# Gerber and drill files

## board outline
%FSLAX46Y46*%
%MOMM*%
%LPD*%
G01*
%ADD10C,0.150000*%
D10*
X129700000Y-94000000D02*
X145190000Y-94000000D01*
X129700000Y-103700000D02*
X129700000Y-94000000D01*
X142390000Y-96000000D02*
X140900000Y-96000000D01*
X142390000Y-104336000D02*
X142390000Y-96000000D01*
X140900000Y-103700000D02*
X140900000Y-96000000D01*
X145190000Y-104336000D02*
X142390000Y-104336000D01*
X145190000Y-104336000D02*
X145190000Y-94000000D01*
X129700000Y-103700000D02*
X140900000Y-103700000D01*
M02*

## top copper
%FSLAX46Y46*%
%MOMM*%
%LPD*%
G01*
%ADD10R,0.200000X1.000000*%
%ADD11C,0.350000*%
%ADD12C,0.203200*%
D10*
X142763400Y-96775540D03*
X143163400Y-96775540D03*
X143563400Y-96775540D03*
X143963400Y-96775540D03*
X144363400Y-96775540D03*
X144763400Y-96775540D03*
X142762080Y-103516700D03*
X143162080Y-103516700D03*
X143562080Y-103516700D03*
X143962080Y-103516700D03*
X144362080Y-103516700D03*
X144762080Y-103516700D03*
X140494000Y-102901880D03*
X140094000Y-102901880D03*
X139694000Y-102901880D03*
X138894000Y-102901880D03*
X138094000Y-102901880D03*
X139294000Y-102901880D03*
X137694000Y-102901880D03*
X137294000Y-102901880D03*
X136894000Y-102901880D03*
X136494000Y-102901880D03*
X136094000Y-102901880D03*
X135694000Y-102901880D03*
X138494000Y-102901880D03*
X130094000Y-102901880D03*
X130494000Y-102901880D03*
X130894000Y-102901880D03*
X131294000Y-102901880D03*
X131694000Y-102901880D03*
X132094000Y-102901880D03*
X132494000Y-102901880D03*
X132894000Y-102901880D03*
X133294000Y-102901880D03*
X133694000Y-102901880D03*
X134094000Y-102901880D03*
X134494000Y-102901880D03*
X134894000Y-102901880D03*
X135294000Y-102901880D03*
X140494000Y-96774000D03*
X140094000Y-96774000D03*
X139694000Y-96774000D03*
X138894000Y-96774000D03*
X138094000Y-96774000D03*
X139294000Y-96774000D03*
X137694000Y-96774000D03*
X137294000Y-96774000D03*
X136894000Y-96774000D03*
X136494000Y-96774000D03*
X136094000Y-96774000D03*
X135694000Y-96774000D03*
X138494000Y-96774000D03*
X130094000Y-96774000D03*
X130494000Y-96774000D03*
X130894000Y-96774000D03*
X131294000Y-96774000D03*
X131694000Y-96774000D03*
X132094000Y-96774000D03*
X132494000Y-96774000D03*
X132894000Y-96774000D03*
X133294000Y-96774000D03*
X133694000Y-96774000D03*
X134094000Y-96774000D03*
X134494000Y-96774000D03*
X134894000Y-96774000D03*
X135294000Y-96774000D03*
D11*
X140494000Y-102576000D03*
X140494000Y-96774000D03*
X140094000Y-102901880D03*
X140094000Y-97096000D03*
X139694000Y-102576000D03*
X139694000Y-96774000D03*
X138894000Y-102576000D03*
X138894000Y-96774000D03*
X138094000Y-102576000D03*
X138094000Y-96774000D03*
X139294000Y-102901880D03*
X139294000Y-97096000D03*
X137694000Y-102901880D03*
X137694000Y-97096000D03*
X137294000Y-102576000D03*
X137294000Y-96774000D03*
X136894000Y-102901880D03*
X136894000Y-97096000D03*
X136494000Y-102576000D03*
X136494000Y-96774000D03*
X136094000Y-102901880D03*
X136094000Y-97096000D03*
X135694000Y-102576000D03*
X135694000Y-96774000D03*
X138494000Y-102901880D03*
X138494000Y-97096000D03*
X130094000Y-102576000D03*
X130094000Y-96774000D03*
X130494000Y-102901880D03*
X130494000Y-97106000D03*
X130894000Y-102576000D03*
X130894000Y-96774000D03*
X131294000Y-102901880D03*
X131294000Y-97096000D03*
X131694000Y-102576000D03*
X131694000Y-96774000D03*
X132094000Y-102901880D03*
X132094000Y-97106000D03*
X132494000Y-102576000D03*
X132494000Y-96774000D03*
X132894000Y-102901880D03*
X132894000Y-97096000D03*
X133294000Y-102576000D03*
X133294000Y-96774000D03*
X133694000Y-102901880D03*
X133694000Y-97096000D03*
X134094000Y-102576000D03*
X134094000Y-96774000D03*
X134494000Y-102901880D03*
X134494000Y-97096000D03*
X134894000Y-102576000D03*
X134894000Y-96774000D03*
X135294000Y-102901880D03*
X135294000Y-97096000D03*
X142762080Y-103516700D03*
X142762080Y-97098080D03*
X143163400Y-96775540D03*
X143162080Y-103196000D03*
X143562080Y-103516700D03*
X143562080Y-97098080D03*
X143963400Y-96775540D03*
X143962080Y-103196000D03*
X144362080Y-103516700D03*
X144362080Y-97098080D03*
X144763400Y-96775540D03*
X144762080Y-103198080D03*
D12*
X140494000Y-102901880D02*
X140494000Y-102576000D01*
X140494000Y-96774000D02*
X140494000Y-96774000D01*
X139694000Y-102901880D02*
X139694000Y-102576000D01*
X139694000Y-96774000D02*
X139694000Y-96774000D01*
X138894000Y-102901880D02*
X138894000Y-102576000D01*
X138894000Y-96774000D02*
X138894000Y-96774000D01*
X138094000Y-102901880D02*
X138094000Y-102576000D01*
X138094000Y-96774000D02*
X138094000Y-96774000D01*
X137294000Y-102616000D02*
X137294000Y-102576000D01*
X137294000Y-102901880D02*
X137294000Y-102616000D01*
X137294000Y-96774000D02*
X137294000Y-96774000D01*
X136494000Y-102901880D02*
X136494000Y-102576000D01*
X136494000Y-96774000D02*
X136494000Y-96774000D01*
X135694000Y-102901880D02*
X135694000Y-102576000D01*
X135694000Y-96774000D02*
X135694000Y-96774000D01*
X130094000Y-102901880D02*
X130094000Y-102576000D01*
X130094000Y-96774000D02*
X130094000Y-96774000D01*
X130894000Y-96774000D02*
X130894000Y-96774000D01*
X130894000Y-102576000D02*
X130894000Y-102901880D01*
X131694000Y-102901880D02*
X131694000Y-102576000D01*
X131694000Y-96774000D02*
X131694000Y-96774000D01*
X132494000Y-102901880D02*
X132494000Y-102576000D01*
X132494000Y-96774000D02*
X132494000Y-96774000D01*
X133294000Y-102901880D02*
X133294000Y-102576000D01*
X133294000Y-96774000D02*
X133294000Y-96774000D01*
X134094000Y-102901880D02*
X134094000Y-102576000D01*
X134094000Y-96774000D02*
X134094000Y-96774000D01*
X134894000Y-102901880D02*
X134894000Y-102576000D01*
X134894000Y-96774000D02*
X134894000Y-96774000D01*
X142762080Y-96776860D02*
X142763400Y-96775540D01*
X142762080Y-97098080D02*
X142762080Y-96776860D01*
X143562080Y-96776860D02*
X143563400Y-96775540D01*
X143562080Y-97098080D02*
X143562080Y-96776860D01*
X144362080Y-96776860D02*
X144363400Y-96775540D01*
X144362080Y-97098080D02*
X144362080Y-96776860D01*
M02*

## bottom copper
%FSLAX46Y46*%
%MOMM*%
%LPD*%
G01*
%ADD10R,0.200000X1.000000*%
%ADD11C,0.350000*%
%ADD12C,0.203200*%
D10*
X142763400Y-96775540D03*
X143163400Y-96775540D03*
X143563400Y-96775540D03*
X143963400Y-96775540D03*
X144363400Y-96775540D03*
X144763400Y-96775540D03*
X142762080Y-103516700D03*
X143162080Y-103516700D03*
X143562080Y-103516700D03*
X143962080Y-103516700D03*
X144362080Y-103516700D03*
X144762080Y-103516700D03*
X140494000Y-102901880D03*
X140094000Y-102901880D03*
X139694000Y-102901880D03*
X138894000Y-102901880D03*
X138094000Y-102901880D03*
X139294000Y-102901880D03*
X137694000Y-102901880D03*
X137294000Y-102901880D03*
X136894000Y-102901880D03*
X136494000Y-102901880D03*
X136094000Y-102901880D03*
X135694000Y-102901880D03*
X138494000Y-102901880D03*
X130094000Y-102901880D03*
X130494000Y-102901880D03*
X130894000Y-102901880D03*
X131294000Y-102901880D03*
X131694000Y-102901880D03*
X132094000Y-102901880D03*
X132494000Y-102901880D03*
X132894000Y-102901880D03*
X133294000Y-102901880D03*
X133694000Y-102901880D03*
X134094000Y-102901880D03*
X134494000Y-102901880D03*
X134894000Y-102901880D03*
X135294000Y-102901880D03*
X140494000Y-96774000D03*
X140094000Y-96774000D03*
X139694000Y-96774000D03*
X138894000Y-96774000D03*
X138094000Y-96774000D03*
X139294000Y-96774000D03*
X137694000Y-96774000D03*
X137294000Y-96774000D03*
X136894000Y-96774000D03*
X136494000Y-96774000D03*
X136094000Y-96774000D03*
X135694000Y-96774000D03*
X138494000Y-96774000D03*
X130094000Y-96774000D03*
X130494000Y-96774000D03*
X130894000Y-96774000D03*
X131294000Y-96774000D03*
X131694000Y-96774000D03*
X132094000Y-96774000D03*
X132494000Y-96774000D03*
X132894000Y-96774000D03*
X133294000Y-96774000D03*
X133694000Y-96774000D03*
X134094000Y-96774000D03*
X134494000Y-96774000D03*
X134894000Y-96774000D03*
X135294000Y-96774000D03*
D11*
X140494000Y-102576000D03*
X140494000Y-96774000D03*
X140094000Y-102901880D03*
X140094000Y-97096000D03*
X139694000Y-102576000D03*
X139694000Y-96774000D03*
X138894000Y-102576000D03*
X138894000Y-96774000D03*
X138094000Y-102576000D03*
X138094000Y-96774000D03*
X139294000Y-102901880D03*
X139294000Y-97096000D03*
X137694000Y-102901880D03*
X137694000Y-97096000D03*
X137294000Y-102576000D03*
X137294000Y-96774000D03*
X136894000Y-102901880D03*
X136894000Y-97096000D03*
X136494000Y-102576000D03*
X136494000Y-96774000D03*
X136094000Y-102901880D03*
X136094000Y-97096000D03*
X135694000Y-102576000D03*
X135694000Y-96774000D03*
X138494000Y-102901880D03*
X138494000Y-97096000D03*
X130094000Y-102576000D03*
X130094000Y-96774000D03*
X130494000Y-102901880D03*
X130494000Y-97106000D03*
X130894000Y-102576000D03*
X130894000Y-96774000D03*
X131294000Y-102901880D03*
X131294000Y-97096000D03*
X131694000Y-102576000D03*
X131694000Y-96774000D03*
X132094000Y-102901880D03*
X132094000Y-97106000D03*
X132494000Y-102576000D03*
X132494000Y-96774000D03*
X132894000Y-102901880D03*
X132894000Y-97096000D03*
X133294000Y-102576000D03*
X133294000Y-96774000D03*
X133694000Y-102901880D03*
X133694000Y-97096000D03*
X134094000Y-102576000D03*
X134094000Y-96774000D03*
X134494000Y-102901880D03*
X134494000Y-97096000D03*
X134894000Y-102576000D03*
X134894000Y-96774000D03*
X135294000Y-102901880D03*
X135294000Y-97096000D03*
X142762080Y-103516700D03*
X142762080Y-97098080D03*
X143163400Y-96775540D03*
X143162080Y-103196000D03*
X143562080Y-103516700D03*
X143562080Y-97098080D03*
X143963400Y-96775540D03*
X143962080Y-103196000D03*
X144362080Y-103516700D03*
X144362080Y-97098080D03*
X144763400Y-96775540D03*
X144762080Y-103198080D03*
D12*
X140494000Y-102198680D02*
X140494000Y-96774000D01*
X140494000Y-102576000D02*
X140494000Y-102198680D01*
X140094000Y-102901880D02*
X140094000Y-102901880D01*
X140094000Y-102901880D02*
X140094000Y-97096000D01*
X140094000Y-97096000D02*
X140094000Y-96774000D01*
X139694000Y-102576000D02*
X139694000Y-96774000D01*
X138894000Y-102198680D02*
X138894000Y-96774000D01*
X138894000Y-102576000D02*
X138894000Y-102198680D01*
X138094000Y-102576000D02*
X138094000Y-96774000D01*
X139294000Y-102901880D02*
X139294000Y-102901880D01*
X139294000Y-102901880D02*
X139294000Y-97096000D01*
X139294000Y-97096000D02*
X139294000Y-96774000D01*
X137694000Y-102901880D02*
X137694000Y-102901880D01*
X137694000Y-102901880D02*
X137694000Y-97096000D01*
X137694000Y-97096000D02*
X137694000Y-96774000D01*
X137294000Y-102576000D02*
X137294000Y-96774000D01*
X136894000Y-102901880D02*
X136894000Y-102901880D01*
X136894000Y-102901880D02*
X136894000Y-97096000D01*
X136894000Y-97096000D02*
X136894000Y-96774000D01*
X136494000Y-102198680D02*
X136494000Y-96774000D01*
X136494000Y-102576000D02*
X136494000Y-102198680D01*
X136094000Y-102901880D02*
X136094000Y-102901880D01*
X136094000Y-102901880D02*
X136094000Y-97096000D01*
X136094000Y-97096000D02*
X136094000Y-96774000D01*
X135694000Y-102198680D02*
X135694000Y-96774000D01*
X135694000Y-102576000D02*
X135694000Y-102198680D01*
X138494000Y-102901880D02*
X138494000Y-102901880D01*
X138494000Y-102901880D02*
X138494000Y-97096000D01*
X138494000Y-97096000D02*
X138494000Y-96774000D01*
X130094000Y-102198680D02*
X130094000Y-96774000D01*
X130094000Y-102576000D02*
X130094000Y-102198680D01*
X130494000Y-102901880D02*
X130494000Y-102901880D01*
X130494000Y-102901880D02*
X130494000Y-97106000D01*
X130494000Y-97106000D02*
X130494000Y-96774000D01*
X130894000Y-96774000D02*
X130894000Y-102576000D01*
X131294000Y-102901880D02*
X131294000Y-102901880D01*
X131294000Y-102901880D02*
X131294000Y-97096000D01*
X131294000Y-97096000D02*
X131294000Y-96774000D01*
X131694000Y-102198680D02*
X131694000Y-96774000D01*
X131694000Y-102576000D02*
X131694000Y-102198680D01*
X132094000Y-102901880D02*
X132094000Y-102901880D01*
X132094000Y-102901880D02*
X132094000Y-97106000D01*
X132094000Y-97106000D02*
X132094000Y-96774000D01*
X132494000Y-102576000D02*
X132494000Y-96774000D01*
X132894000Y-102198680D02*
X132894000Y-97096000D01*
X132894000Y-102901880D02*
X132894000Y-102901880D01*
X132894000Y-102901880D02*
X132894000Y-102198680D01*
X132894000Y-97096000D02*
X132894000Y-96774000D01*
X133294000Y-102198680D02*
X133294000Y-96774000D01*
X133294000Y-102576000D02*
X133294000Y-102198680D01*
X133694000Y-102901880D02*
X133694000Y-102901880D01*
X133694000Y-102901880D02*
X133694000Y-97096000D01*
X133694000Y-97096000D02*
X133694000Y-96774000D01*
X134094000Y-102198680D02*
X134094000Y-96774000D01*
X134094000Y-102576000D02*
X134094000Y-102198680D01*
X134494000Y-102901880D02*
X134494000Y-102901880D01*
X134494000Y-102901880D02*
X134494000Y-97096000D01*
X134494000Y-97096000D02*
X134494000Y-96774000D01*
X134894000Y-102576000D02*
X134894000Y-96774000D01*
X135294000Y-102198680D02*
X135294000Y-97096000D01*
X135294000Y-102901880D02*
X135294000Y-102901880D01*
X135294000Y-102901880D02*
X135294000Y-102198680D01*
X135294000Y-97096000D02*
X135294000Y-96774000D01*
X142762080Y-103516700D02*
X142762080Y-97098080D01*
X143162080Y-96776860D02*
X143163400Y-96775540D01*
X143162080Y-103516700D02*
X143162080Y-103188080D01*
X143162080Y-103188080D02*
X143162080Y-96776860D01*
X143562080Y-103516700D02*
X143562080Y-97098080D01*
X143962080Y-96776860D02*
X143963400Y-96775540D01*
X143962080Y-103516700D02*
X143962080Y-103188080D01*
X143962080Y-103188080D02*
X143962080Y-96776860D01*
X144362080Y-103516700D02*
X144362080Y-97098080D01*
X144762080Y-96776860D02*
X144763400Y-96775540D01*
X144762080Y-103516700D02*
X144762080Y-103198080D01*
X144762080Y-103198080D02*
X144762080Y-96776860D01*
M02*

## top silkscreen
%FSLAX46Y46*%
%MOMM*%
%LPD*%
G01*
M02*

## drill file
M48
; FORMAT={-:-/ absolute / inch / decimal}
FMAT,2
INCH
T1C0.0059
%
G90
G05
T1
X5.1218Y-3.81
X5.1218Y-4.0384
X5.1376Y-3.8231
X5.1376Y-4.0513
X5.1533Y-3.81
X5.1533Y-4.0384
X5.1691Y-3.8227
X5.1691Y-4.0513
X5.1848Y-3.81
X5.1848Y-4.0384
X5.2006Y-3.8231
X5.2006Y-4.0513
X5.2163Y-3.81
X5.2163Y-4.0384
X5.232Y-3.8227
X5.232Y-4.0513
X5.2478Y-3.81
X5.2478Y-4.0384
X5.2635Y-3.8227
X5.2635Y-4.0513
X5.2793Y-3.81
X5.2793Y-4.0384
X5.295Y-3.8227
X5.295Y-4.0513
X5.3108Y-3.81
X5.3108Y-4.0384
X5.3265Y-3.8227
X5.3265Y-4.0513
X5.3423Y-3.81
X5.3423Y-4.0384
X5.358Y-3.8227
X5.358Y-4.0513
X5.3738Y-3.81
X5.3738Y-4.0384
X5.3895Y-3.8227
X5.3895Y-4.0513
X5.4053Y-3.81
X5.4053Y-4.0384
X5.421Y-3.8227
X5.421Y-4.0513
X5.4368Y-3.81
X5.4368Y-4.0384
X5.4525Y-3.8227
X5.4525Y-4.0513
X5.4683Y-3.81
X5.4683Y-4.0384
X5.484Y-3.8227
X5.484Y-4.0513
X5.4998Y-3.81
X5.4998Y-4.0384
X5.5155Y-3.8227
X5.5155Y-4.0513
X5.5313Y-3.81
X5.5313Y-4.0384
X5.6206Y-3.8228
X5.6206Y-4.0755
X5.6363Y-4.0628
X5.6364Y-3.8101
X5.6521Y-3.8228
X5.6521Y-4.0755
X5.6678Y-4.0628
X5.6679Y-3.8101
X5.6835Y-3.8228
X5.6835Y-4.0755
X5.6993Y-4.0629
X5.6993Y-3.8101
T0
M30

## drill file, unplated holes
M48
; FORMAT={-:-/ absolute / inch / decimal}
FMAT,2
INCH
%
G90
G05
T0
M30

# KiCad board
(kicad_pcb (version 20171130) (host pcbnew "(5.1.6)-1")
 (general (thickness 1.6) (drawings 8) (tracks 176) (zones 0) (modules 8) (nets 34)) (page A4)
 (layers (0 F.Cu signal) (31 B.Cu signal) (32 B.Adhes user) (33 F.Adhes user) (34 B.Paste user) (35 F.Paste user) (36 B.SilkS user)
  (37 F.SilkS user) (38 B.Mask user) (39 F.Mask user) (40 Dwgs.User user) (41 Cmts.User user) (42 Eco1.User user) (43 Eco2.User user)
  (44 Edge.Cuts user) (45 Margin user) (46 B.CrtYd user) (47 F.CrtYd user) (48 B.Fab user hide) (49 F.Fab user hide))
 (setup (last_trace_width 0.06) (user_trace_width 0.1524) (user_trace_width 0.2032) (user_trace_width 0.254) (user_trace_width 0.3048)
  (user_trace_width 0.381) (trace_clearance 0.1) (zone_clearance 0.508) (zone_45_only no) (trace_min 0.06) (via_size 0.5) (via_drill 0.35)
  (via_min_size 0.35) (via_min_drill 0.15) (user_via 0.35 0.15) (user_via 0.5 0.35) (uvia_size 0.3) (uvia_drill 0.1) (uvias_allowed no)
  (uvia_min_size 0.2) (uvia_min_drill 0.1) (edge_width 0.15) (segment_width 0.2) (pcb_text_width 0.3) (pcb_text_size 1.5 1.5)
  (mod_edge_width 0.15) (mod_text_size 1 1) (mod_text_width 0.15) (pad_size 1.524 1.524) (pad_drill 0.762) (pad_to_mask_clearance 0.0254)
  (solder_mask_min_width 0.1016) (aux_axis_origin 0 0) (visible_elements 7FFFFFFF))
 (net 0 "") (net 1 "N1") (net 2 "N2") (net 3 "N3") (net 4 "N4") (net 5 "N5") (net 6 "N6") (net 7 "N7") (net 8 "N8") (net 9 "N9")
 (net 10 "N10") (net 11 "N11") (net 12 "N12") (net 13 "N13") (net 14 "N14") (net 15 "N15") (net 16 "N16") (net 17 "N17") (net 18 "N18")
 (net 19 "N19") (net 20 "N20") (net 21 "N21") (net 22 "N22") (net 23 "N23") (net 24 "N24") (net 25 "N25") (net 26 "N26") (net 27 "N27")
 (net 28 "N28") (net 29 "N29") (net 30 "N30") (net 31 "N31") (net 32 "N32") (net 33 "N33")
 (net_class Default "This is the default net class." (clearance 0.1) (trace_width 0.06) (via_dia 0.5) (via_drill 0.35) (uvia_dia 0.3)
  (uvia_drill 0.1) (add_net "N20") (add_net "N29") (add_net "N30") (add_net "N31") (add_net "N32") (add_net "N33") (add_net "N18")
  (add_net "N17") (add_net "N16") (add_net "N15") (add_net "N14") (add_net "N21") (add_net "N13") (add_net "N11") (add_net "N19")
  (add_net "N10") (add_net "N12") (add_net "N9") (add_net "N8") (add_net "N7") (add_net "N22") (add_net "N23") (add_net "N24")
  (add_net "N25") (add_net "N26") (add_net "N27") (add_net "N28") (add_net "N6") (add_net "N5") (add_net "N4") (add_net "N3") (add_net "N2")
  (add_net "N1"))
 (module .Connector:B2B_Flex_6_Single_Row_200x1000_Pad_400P (layer F.Cu) (at 144.7634 96.77554 180)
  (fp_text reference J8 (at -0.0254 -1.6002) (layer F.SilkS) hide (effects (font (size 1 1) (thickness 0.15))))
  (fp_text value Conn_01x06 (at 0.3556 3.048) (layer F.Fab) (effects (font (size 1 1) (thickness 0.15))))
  (pad 6 smd rect (at 2 0 180) (size 0.2 1) (layers F.Cu F.Paste F.Mask) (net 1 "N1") (zone_connect 0))
  (pad 5 smd rect (at 1.6 0 180) (size 0.2 1) (layers F.Cu F.Paste F.Mask) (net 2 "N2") (zone_connect 0))
  (pad 4 smd rect (at 1.2 0 180) (size 0.2 1) (layers F.Cu F.Paste F.Mask) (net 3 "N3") (zone_connect 0))
  (pad 3 smd rect (at 0.8 0 180) (size 0.2 1) (layers F.Cu F.Paste F.Mask) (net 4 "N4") (zone_connect 0))
  (pad 2 smd rect (at 0.4 0 180) (size 0.2 1) (layers F.Cu F.Paste F.Mask) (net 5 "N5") (zone_connect 0))
  (pad 1 smd rect (at 0 0 180) (size 0.2 1) (layers F.Cu F.Paste F.Mask) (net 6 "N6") (zone_connect 0)))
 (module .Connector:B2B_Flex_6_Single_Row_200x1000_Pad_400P (layer F.Cu) (at 144.76208 103.5167 180)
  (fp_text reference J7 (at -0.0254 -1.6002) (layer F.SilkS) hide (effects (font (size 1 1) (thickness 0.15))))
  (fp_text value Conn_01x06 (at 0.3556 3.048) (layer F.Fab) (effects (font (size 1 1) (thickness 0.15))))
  (pad 6 smd rect (at 2 0 180) (size 0.2 1) (layers F.Cu F.Paste F.Mask) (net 1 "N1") (zone_connect 0))
  (pad 5 smd rect (at 1.6 0 180) (size 0.2 1) (layers F.Cu F.Paste F.Mask) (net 2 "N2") (zone_connect 0))
  (pad 4 smd rect (at 1.2 0 180) (size 0.2 1) (layers F.Cu F.Paste F.Mask) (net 3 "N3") (zone_connect 0))
  (pad 3 smd rect (at 0.8 0 180) (size 0.2 1) (layers F.Cu F.Paste F.Mask) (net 4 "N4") (zone_connect 0))
  (pad 2 smd rect (at 0.4 0 180) (size 0.2 1) (layers F.Cu F.Paste F.Mask) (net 5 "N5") (zone_connect 0))
  (pad 1 smd rect (at 0 0 180) (size 0.2 1) (layers F.Cu F.Paste F.Mask) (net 6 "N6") (zone_connect 0)))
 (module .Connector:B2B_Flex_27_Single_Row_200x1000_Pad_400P (layer F.Cu) (at 130.094 102.90188)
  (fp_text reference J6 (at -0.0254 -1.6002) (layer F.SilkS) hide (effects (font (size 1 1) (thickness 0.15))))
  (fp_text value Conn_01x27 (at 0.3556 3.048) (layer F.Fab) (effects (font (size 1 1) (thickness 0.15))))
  (pad 27 smd rect (at 10.4 0) (size 0.2 1) (layers F.Cu F.Paste F.Mask) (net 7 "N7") (zone_connect 0))
  (pad 26 smd rect (at 10 0) (size 0.2 1) (layers F.Cu F.Paste F.Mask) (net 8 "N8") (zone_connect 0))
  (pad 25 smd rect (at 9.6 0) (size 0.2 1) (layers F.Cu F.Paste F.Mask) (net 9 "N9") (zone_connect 0))
  (pad 23 smd rect (at 8.8 0) (size 0.2 1) (layers F.Cu F.Paste F.Mask) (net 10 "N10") (zone_connect 0))
  (pad 21 smd rect (at 8 0) (size 0.2 1) (layers F.Cu F.Paste F.Mask) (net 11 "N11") (zone_connect 0))
  (pad 24 smd rect (at 9.2 0) (size 0.2 1) (layers F.Cu F.Paste F.Mask) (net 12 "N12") (zone_connect 0))
  (pad 20 smd rect (at 7.6 0) (size 0.2 1) (layers F.Cu F.Paste F.Mask) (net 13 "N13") (zone_connect 0))
  (pad 19 smd rect (at 7.2 0) (size 0.2 1) (layers F.Cu F.Paste F.Mask) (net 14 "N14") (zone_connect 0))
  (pad 18 smd rect (at 6.8 0) (size 0.2 1) (layers F.Cu F.Paste F.Mask) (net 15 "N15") (zone_connect 0))
  (pad 17 smd rect (at 6.4 0) (size 0.2 1) (layers F.Cu F.Paste F.Mask) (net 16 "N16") (zone_connect 0))
  (pad 16 smd rect (at 6 0) (size 0.2 1) (layers F.Cu F.Paste F.Mask) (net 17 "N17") (zone_connect 0))
  (pad 15 smd rect (at 5.6 0) (size 0.2 1) (layers F.Cu F.Paste F.Mask) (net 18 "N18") (zone_connect 0))
  (pad 22 smd rect (at 8.4 0) (size 0.2 1) (layers F.Cu F.Paste F.Mask) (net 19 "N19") (zone_connect 0))
  (pad 1 smd rect (at 0 0) (size 0.2 1) (layers F.Cu F.Paste F.Mask) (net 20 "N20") (zone_connect 0))
  (pad 2 smd rect (at 0.4 0) (size 0.2 1) (layers F.Cu F.Paste F.Mask) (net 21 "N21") (zone_connect 0))
  (pad 3 smd rect (at 0.8 0) (size 0.2 1) (layers F.Cu F.Paste F.Mask) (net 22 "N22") (zone_connect 0))
  (pad 4 smd rect (at 1.2 0) (size 0.2 1) (layers F.Cu F.Paste F.Mask) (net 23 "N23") (zone_connect 0))
  (pad 5 smd rect (at 1.6 0) (size 0.2 1) (layers F.Cu F.Paste F.Mask) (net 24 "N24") (zone_connect 0))
  (pad 6 smd rect (at 2 0) (size 0.2 1) (layers F.Cu F.Paste F.Mask) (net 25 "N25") (zone_connect 0))
  (pad 7 smd rect (at 2.4 0) (size 0.2 1) (layers F.Cu F.Paste F.Mask) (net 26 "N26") (zone_connect 0))
  (pad 8 smd rect (at 2.8 0) (size 0.2 1) (layers F.Cu F.Paste F.Mask) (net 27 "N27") (zone_connect 0))
  (pad 9 smd rect (at 3.2 0) (size 0.2 1) (layers F.Cu F.Paste F.Mask) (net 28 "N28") (zone_connect 0))
  (pad 10 smd rect (at 3.6 0) (size 0.2 1) (layers F.Cu F.Paste F.Mask) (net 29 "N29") (zone_connect 0))
  (pad 11 smd rect (at 4 0) (size 0.2 1) (layers F.Cu F.Paste F.Mask) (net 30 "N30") (zone_connect 0))
  (pad 12 smd rect (at 4.4 0) (size 0.2 1) (layers F.Cu F.Paste F.Mask) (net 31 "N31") (zone_connect 0))
  (pad 13 smd rect (at 4.8 0) (size 0.2 1) (layers F.Cu F.Paste F.Mask) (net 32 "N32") (zone_connect 0))
  (pad 14 smd rect (at 5.2 0) (size 0.2 1) (layers F.Cu F.Paste F.Mask) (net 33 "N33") (zone_connect 0)))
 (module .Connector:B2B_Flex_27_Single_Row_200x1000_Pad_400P (layer F.Cu) (at 130.094 96.774)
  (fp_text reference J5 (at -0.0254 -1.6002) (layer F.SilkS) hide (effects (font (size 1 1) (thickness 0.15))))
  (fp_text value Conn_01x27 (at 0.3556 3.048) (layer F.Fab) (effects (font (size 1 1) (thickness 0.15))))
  (pad 27 smd rect (at 10.4 0) (size 0.2 1) (layers F.Cu F.Paste F.Mask) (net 7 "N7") (zone_connect 0))
  (pad 26 smd rect (at 10 0) (size 0.2 1) (layers F.Cu F.Paste F.Mask) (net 8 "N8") (zone_connect 0))
  (pad 25 smd rect (at 9.6 0) (size 0.2 1) (layers F.Cu F.Paste F.Mask) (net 9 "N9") (zone_connect 0))
  (pad 23 smd rect (at 8.8 0) (size 0.2 1) (layers F.Cu F.Paste F.Mask) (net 10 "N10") (zone_connect 0))
  (pad 21 smd rect (at 8 0) (size 0.2 1) (layers F.Cu F.Paste F.Mask) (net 11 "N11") (zone_connect 0))
  (pad 24 smd rect (at 9.2 0) (size 0.2 1) (layers F.Cu F.Paste F.Mask) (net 12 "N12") (zone_connect 0))
  (pad 20 smd rect (at 7.6 0) (size 0.2 1) (layers F.Cu F.Paste F.Mask) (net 13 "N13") (zone_connect 0))
  (pad 19 smd rect (at 7.2 0) (size 0.2 1) (layers F.Cu F.Paste F.Mask) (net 14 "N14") (zone_connect 0))
  (pad 18 smd rect (at 6.8 0) (size 0.2 1) (layers F.Cu F.Paste F.Mask) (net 15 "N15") (zone_connect 0))
  (pad 17 smd rect (at 6.4 0) (size 0.2 1) (layers F.Cu F.Paste F.Mask) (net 16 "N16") (zone_connect 0))
  (pad 16 smd rect (at 6 0) (size 0.2 1) (layers F.Cu F.Paste F.Mask) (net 17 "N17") (zone_connect 0))
  (pad 15 smd rect (at 5.6 0) (size 0.2 1) (layers F.Cu F.Paste F.Mask) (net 18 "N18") (zone_connect 0))
  (pad 22 smd rect (at 8.4 0) (size 0.2 1) (layers F.Cu F.Paste F.Mask) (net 19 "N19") (zone_connect 0))
  (pad 1 smd rect (at 0 0) (size 0.2 1) (layers F.Cu F.Paste F.Mask) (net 20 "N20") (zone_connect 0))
  (pad 2 smd rect (at 0.4 0) (size 0.2 1) (layers F.Cu F.Paste F.Mask) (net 21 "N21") (zone_connect 0))
  (pad 3 smd rect (at 0.8 0) (size 0.2 1) (layers F.Cu F.Paste F.Mask) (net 22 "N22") (zone_connect 0))
  (pad 4 smd rect (at 1.2 0) (size 0.2 1) (layers F.Cu F.Paste F.Mask) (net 23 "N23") (zone_connect 0))
  (pad 5 smd rect (at 1.6 0) (size 0.2 1) (layers F.Cu F.Paste F.Mask) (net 24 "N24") (zone_connect 0))
  (pad 6 smd rect (at 2 0) (size 0.2 1) (layers F.Cu F.Paste F.Mask) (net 25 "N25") (zone_connect 0))
  (pad 7 smd rect (at 2.4 0) (size 0.2 1) (layers F.Cu F.Paste F.Mask) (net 26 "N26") (zone_connect 0))
  (pad 8 smd rect (at 2.8 0) (size 0.2 1) (layers F.Cu F.Paste F.Mask) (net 27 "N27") (zone_connect 0))
  (pad 9 smd rect (at 3.2 0) (size 0.2 1) (layers F.Cu F.Paste F.Mask) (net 28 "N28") (zone_connect 0))
  (pad 10 smd rect (at 3.6 0) (size 0.2 1) (layers F.Cu F.Paste F.Mask) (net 29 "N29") (zone_connect 0))
  (pad 11 smd rect (at 4 0) (size 0.2 1) (layers F.Cu F.Paste F.Mask) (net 30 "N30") (zone_connect 0))
  (pad 12 smd rect (at 4.4 0) (size 0.2 1) (layers F.Cu F.Paste F.Mask) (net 31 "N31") (zone_connect 0))
  (pad 13 smd rect (at 4.8 0) (size 0.2 1) (layers F.Cu F.Paste F.Mask) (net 32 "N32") (zone_connect 0))
  (pad 14 smd rect (at 5.2 0) (size 0.2 1) (layers F.Cu F.Paste F.Mask) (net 33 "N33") (zone_connect 0)))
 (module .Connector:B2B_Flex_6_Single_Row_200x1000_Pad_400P (layer B.Cu) (at 144.7634 96.77554 180)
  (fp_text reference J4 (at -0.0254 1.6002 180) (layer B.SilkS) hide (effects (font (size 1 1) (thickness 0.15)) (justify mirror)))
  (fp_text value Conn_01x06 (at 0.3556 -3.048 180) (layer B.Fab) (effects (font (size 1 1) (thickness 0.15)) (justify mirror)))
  (pad 6 smd rect (at 2 0 180) (size 0.2 1) (layers B.Cu B.Paste B.Mask) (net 1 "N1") (zone_connect 0))
  (pad 5 smd rect (at 1.6 0 180) (size 0.2 1) (layers B.Cu B.Paste B.Mask) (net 2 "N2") (zone_connect 0))
  (pad 4 smd rect (at 1.2 0 180) (size 0.2 1) (layers B.Cu B.Paste B.Mask) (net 3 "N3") (zone_connect 0))
  (pad 3 smd rect (at 0.8 0 180) (size 0.2 1) (layers B.Cu B.Paste B.Mask) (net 4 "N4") (zone_connect 0))
  (pad 2 smd rect (at 0.4 0 180) (size 0.2 1) (layers B.Cu B.Paste B.Mask) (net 5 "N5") (zone_connect 0))
  (pad 1 smd rect (at 0 0 180) (size 0.2 1) (layers B.Cu B.Paste B.Mask) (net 6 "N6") (zone_connect 0)))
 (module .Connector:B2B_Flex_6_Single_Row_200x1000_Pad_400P (layer B.Cu) (at 144.76208 103.5167 180)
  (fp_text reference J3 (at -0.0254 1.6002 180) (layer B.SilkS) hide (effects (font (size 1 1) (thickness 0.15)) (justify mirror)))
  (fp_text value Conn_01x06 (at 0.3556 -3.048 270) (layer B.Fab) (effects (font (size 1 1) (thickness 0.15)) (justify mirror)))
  (pad 6 smd rect (at 2 0 180) (size 0.2 1) (layers B.Cu B.Paste B.Mask) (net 1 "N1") (zone_connect 0))
  (pad 5 smd rect (at 1.6 0 180) (size 0.2 1) (layers B.Cu B.Paste B.Mask) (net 2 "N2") (zone_connect 0))
  (pad 4 smd rect (at 1.2 0 180) (size 0.2 1) (layers B.Cu B.Paste B.Mask) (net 3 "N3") (zone_connect 0))
  (pad 3 smd rect (at 0.8 0 180) (size 0.2 1) (layers B.Cu B.Paste B.Mask) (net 4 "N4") (zone_connect 0))
  (pad 2 smd rect (at 0.4 0 180) (size 0.2 1) (layers B.Cu B.Paste B.Mask) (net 5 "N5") (zone_connect 0))
  (pad 1 smd rect (at 0 0 180) (size 0.2 1) (layers B.Cu B.Paste B.Mask) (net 6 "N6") (zone_connect 0)))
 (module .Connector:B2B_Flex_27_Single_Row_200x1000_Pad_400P (layer B.Cu) (at 130.094 102.90188)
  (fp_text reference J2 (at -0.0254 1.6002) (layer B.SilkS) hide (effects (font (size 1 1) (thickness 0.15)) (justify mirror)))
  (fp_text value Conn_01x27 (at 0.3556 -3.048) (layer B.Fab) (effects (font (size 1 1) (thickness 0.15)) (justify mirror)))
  (pad 27 smd rect (at 10.4 0) (size 0.2 1) (layers B.Cu B.Paste B.Mask) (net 7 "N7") (zone_connect 0))
  (pad 26 smd rect (at 10 0) (size 0.2 1) (layers B.Cu B.Paste B.Mask) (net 8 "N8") (zone_connect 0))
  (pad 25 smd rect (at 9.6 0) (size 0.2 1) (layers B.Cu B.Paste B.Mask) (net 9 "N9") (zone_connect 0))
  (pad 23 smd rect (at 8.8 0) (size 0.2 1) (layers B.Cu B.Paste B.Mask) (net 10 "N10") (zone_connect 0))
  (pad 21 smd rect (at 8 0) (size 0.2 1) (layers B.Cu B.Paste B.Mask) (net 11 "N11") (zone_connect 0))
  (pad 24 smd rect (at 9.2 0) (size 0.2 1) (layers B.Cu B.Paste B.Mask) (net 12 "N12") (zone_connect 0))
  (pad 20 smd rect (at 7.6 0) (size 0.2 1) (layers B.Cu B.Paste B.Mask) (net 13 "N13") (zone_connect 0))
  (pad 19 smd rect (at 7.2 0) (size 0.2 1) (layers B.Cu B.Paste B.Mask) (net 14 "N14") (zone_connect 0))
  (pad 18 smd rect (at 6.8 0) (size 0.2 1) (layers B.Cu B.Paste B.Mask) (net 15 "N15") (zone_connect 0))
  (pad 17 smd rect (at 6.4 0) (size 0.2 1) (layers B.Cu B.Paste B.Mask) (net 16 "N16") (zone_connect 0))
  (pad 16 smd rect (at 6 0) (size 0.2 1) (layers B.Cu B.Paste B.Mask) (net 17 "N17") (zone_connect 0))
  (pad 15 smd rect (at 5.6 0) (size 0.2 1) (layers B.Cu B.Paste B.Mask) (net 18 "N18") (zone_connect 0))
  (pad 22 smd rect (at 8.4 0) (size 0.2 1) (layers B.Cu B.Paste B.Mask) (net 19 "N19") (zone_connect 0))
  (pad 1 smd rect (at 0 0) (size 0.2 1) (layers B.Cu B.Paste B.Mask) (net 20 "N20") (zone_connect 0))
  (pad 2 smd rect (at 0.4 0) (size 0.2 1) (layers B.Cu B.Paste B.Mask) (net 21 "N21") (zone_connect 0))
  (pad 3 smd rect (at 0.8 0) (size 0.2 1) (layers B.Cu B.Paste B.Mask) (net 22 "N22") (zone_connect 0))
  (pad 4 smd rect (at 1.2 0) (size 0.2 1) (layers B.Cu B.Paste B.Mask) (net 23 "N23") (zone_connect 0))
  (pad 5 smd rect (at 1.6 0) (size 0.2 1) (layers B.Cu B.Paste B.Mask) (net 24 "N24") (zone_connect 0))
  (pad 6 smd rect (at 2 0) (size 0.2 1) (layers B.Cu B.Paste B.Mask) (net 25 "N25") (zone_connect 0))
  (pad 7 smd rect (at 2.4 0) (size 0.2 1) (layers B.Cu B.Paste B.Mask) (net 26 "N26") (zone_connect 0))
  (pad 8 smd rect (at 2.8 0) (size 0.2 1) (layers B.Cu B.Paste B.Mask) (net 27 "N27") (zone_connect 0))
  (pad 9 smd rect (at 3.2 0) (size 0.2 1) (layers B.Cu B.Paste B.Mask) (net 28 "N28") (zone_connect 0))
  (pad 10 smd rect (at 3.6 0) (size 0.2 1) (layers B.Cu B.Paste B.Mask) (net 29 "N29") (zone_connect 0))
  (pad 11 smd rect (at 4 0) (size 0.2 1) (layers B.Cu B.Paste B.Mask) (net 30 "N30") (zone_connect 0))
  (pad 12 smd rect (at 4.4 0) (size 0.2 1) (layers B.Cu B.Paste B.Mask) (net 31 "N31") (zone_connect 0))
  (pad 13 smd rect (at 4.8 0) (size 0.2 1) (layers B.Cu B.Paste B.Mask) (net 32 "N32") (zone_connect 0))
  (pad 14 smd rect (at 5.2 0) (size 0.2 1) (layers B.Cu B.Paste B.Mask) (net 33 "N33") (zone_connect 0)))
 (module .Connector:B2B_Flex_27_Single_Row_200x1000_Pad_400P (layer B.Cu) (at 130.094 96.774)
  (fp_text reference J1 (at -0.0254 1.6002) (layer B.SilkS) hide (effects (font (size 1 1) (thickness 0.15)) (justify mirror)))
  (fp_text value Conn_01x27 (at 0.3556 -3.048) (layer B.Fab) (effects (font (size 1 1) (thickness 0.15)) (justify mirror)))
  (pad 27 smd rect (at 10.4 0) (size 0.2 1) (layers B.Cu B.Paste B.Mask) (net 7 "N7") (zone_connect 0))
  (pad 26 smd rect (at 10 0) (size 0.2 1) (layers B.Cu B.Paste B.Mask) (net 8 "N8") (zone_connect 0))
  (pad 25 smd rect (at 9.6 0) (size 0.2 1) (layers B.Cu B.Paste B.Mask) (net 9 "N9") (zone_connect 0))
  (pad 23 smd rect (at 8.8 0) (size 0.2 1) (layers B.Cu B.Paste B.Mask) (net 10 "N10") (zone_connect 0))
  (pad 21 smd rect (at 8 0) (size 0.2 1) (layers B.Cu B.Paste B.Mask) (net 11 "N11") (zone_connect 0))
  (pad 24 smd rect (at 9.2 0) (size 0.2 1) (layers B.Cu B.Paste B.Mask) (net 12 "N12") (zone_connect 0))
  (pad 20 smd rect (at 7.6 0) (size 0.2 1) (layers B.Cu B.Paste B.Mask) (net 13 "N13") (zone_connect 0))
  (pad 19 smd rect (at 7.2 0) (size 0.2 1) (layers B.Cu B.Paste B.Mask) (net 14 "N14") (zone_connect 0))
  (pad 18 smd rect (at 6.8 0) (size 0.2 1) (layers B.Cu B.Paste B.Mask) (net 15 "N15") (zone_connect 0))
  (pad 17 smd rect (at 6.4 0) (size 0.2 1) (layers B.Cu B.Paste B.Mask) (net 16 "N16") (zone_connect 0))
  (pad 16 smd rect (at 6 0) (size 0.2 1) (layers B.Cu B.Paste B.Mask) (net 17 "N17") (zone_connect 0))
  (pad 15 smd rect (at 5.6 0) (size 0.2 1) (layers B.Cu B.Paste B.Mask) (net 18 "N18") (zone_connect 0))
  (pad 22 smd rect (at 8.4 0) (size 0.2 1) (layers B.Cu B.Paste B.Mask) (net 19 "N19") (zone_connect 0))
  (pad 1 smd rect (at 0 0) (size 0.2 1) (layers B.Cu B.Paste B.Mask) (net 20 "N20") (zone_connect 0))
  (pad 2 smd rect (at 0.4 0) (size 0.2 1) (layers B.Cu B.Paste B.Mask) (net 21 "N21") (zone_connect 0))
  (pad 3 smd rect (at 0.8 0) (size 0.2 1) (layers B.Cu B.Paste B.Mask) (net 22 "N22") (zone_connect 0))
  (pad 4 smd rect (at 1.2 0) (size 0.2 1) (layers B.Cu B.Paste B.Mask) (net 23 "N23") (zone_connect 0))
  (pad 5 smd rect (at 1.6 0) (size 0.2 1) (layers B.Cu B.Paste B.Mask) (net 24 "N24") (zone_connect 0))
  (pad 6 smd rect (at 2 0) (size 0.2 1) (layers B.Cu B.Paste B.Mask) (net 25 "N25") (zone_connect 0))
  (pad 7 smd rect (at 2.4 0) (size 0.2 1) (layers B.Cu B.Paste B.Mask) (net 26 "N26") (zone_connect 0))
  (pad 8 smd rect (at 2.8 0) (size 0.2 1) (layers B.Cu B.Paste B.Mask) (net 27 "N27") (zone_connect 0))
  (pad 9 smd rect (at 3.2 0) (size 0.2 1) (layers B.Cu B.Paste B.Mask) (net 28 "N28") (zone_connect 0))
  (pad 10 smd rect (at 3.6 0) (size 0.2 1) (layers B.Cu B.Paste B.Mask) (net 29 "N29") (zone_connect 0))
  (pad 11 smd rect (at 4 0) (size 0.2 1) (layers B.Cu B.Paste B.Mask) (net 30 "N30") (zone_connect 0))
  (pad 12 smd rect (at 4.4 0) (size 0.2 1) (layers B.Cu B.Paste B.Mask) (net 31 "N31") (zone_connect 0))
  (pad 13 smd rect (at 4.8 0) (size 0.2 1) (layers B.Cu B.Paste B.Mask) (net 32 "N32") (zone_connect 0))
  (pad 14 smd rect (at 5.2 0) (size 0.2 1) (layers B.Cu B.Paste B.Mask) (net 33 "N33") (zone_connect 0)))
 (gr_line (start 129.7 94) (end 145.19 94) (layer Edge.Cuts) (width 0.15))
 (gr_line (start 129.7 103.7) (end 129.7 94) (layer Edge.Cuts) (width 0.15))
 (gr_line (start 142.39 96) (end 140.9 96) (layer Edge.Cuts) (width 0.15))
 (gr_line (start 142.39 104.336) (end 142.39 96) (layer Edge.Cuts) (width 0.15))
 (gr_line (start 140.9 103.7) (end 140.9 96) (layer Edge.Cuts) (width 0.15))
 (gr_line (start 145.19 104.336) (end 142.39 104.336) (layer Edge.Cuts) (width 0.15))
 (gr_line (start 145.19 104.336) (end 145.19 94) (layer Edge.Cuts) (width 0.15))
 (gr_line (start 129.7 103.7) (end 140.9 103.7) (layer Edge.Cuts) (width 0.15))
 (segment (start 140.494 102.19868) (end 140.494 96.774) (width 0.2032) (layer B.Cu) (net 7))
 (segment (start 140.494 102.90188) (end 140.494 102.576) (width 0.2032) (layer F.Cu) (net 7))
 (segment (start 140.494 102.576) (end 140.494 102.19868) (width 0.2032) (layer B.Cu) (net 7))
 (via (at 140.494 102.576) (size 0.35) (drill 0.15) (layers F.Cu B.Cu) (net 7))
 (segment (start 140.494 96.774) (end 140.494 96.774) (width 0.2032) (layer F.Cu) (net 7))
 (via (at 140.494 96.774) (size 0.35) (drill 0.15) (layers F.Cu B.Cu) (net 7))
 (segment (start 140.094 102.90188) (end 140.094 102.90188) (width 0.2032) (layer B.Cu) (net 8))
 (segment (start 140.094 102.90188) (end 140.094 97.096) (width 0.2032) (layer B.Cu) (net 8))
 (via (at 140.094 102.90188) (size 0.35) (drill 0.15) (layers F.Cu B.Cu) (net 8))
 (segment (start 140.094 97.096) (end 140.094 96.774) (width 0.2032) (layer B.Cu) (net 8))
 (via (at 140.094 97.096) (size 0.35) (drill 0.15) (layers F.Cu B.Cu) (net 8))
 (segment (start 139.694 102.90188) (end 139.694 102.576) (width 0.2032) (layer F.Cu) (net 9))
 (segment (start 139.694 102.576) (end 139.694 96.774) (width 0.2032) (layer B.Cu) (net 9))
 (via (at 139.694 102.576) (size 0.35) (drill 0.15) (layers F.Cu B.Cu) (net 9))
 (segment (start 139.694 96.774) (end 139.694 96.774) (width 0.2032) (layer F.Cu) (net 9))
 (via (at 139.694 96.774) (size 0.35) (drill 0.15) (layers F.Cu B.Cu) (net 9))
 (segment (start 138.894 102.19868) (end 138.894 96.774) (width 0.2032) (layer B.Cu) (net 10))
 (segment (start 138.894 102.90188) (end 138.894 102.576) (width 0.2032) (layer F.Cu) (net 10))
 (segment (start 138.894 102.576) (end 138.894 102.19868) (width 0.2032) (layer B.Cu) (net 10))
 (via (at 138.894 102.576) (size 0.35) (drill 0.15) (layers F.Cu B.Cu) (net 10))
 (segment (start 138.894 96.774) (end 138.894 96.774) (width 0.2032) (layer F.Cu) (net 10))
 (via (at 138.894 96.774) (size 0.35) (drill 0.15) (layers F.Cu B.Cu) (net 10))
 (segment (start 138.094 102.90188) (end 138.094 102.576) (width 0.2032) (layer F.Cu) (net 11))
 (segment (start 138.094 102.576) (end 138.094 96.774) (width 0.2032) (layer B.Cu) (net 11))
 (via (at 138.094 102.576) (size 0.35) (drill 0.15) (layers F.Cu B.Cu) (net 11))
 (segment (start 138.094 96.774) (end 138.094 96.774) (width 0.2032) (layer F.Cu) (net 11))
 (via (at 138.094 96.774) (size 0.35) (drill 0.15) (layers F.Cu B.Cu) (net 11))
 (segment (start 139.294 102.90188) (end 139.294 102.90188) (width 0.2032) (layer B.Cu) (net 12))
 (segment (start 139.294 102.90188) (end 139.294 97.096) (width 0.2032) (layer B.Cu) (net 12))
 (via (at 139.294 102.90188) (size 0.35) (drill 0.15) (layers F.Cu B.Cu) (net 12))
 (segment (start 139.294 97.096) (end 139.294 96.774) (width 0.2032) (layer B.Cu) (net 12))
 (via (at 139.294 97.096) (size 0.35) (drill 0.15) (layers F.Cu B.Cu) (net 12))
 (segment (start 137.694 102.90188) (end 137.694 102.90188) (width 0.2032) (layer B.Cu) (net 13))
 (segment (start 137.694 102.90188) (end 137.694 97.096) (width 0.2032) (layer B.Cu) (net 13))
 (via (at 137.694 102.90188) (size 0.35) (drill 0.15) (layers F.Cu B.Cu) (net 13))
 (segment (start 137.694 97.096) (end 137.694 96.774) (width 0.2032) (layer B.Cu) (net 13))
 (via (at 137.694 97.096) (size 0.35) (drill 0.15) (layers F.Cu B.Cu) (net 13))
 (segment (start 137.294 102.616) (end 137.294 102.576) (width 0.2032) (layer F.Cu) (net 14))
 (segment (start 137.294 102.90188) (end 137.294 102.616) (width 0.2032) (layer F.Cu) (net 14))
 (segment (start 137.294 102.576) (end 137.294 96.774) (width 0.2032) (layer B.Cu) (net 14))
 (via (at 137.294 102.576) (size 0.35) (drill 0.15) (layers F.Cu B.Cu) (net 14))
 (segment (start 137.294 96.774) (end 137.294 96.774) (width 0.2032) (layer F.Cu) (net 14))
 (via (at 137.294 96.774) (size 0.35) (drill 0.15) (layers F.Cu B.Cu) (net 14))
 (segment (start 136.894 102.90188) (end 136.894 102.90188) (width 0.2032) (layer B.Cu) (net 15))
 (segment (start 136.894 102.90188) (end 136.894 97.096) (width 0.2032) (layer B.Cu) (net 15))
 (via (at 136.894 102.90188) (size 0.35) (drill 0.15) (layers F.Cu B.Cu) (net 15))
 (segment (start 136.894 97.096) (end 136.894 96.774) (width 0.2032) (layer B.Cu) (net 15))
 (via (at 136.894 97.096) (size 0.35) (drill 0.15) (layers F.Cu B.Cu) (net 15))
 (segment (start 136.494 102.19868) (end 136.494 96.774) (width 0.2032) (layer B.Cu) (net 16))
 (segment (start 136.494 102.90188) (end 136.494 102.576) (width 0.2032) (layer F.Cu) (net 16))
 (segment (start 136.494 102.576) (end 136.494 102.19868) (width 0.2032) (layer B.Cu) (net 16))
 (via (at 136.494 102.576) (size 0.35) (drill 0.15) (layers F.Cu B.Cu) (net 16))
 (segment (start 136.494 96.774) (end 136.494 96.774) (width 0.2032) (layer F.Cu) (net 16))
 (via (at 136.494 96.774) (size 0.35) (drill 0.15) (layers F.Cu B.Cu) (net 16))
 (segment (start 136.094 102.90188) (end 136.094 102.90188) (width 0.2032) (layer B.Cu) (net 17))
 (segment (start 136.094 102.90188) (end 136.094 97.096) (width 0.2032) (layer B.Cu) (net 17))
 (via (at 136.094 102.90188) (size 0.35) (drill 0.15) (layers F.Cu B.Cu) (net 17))
 (segment (start 136.094 97.096) (end 136.094 96.774) (width 0.2032) (layer B.Cu) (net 17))
 (via (at 136.094 97.096) (size 0.35) (drill 0.15) (layers F.Cu B.Cu) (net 17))
 (segment (start 135.694 102.19868) (end 135.694 96.774) (width 0.2032) (layer B.Cu) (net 18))
 (segment (start 135.694 102.90188) (end 135.694 102.576) (width 0.2032) (layer F.Cu) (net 18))
 (segment (start 135.694 102.576) (end 135.694 102.19868) (width 0.2032) (layer B.Cu) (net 18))
 (via (at 135.694 102.576) (size 0.35) (drill 0.15) (layers F.Cu B.Cu) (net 18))
 (segment (start 135.694 96.774) (end 135.694 96.774) (width 0.2032) (layer F.Cu) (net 18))
 (via (at 135.694 96.774) (size 0.35) (drill 0.15) (layers F.Cu B.Cu) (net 18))
 (segment (start 138.494 102.90188) (end 138.494 102.90188) (width 0.2032) (layer B.Cu) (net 19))
 (segment (start 138.494 102.90188) (end 138.494 97.096) (width 0.2032) (layer B.Cu) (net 19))
 (via (at 138.494 102.90188) (size 0.35) (drill 0.15) (layers F.Cu B.Cu) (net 19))
 (segment (start 138.494 97.096) (end 138.494 96.774) (width 0.2032) (layer B.Cu) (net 19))
 (via (at 138.494 97.096) (size 0.35) (drill 0.15) (layers F.Cu B.Cu) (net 19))
 (segment (start 130.094 102.19868) (end 130.094 96.774) (width 0.2032) (layer B.Cu) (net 20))
 (segment (start 130.094 102.90188) (end 130.094 102.576) (width 0.2032) (layer F.Cu) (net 20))
 (segment (start 130.094 102.576) (end 130.094 102.19868) (width 0.2032) (layer B.Cu) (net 20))
 (via (at 130.094 102.576) (size 0.35) (drill 0.15) (layers F.Cu B.Cu) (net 20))
 (segment (start 130.094 96.774) (end 130.094 96.774) (width 0.2032) (layer F.Cu) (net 20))
 (via (at 130.094 96.774) (size 0.35) (drill 0.15) (layers F.Cu B.Cu) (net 20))
 (segment (start 130.494 102.90188) (end 130.494 102.90188) (width 0.2032) (layer B.Cu) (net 21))
 (segment (start 130.494 102.90188) (end 130.494 97.106) (width 0.2032) (layer B.Cu) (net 21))
 (via (at 130.494 102.90188) (size 0.35) (drill 0.15) (layers F.Cu B.Cu) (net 21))
 (segment (start 130.494 97.106) (end 130.494 96.774) (width 0.2032) (layer B.Cu) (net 21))
 (via (at 130.494 97.106) (size 0.35) (drill 0.15) (layers F.Cu B.Cu) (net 21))
 (segment (start 130.894 96.774) (end 130.894 96.774) (width 0.2032) (layer F.Cu) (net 22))
 (segment (start 130.894 102.576) (end 130.894 102.90188) (width 0.2032) (layer F.Cu) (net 22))
 (via (at 130.894 102.576) (size 0.35) (drill 0.15) (layers F.Cu B.Cu) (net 22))
 (segment (start 130.894 96.774) (end 130.894 102.576) (width 0.2032) (layer B.Cu) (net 22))
 (via (at 130.894 96.774) (size 0.35) (drill 0.15) (layers F.Cu B.Cu) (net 22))
 (segment (start 131.294 102.90188) (end 131.294 102.90188) (width 0.2032) (layer B.Cu) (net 23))
 (segment (start 131.294 102.90188) (end 131.294 97.096) (width 0.2032) (layer B.Cu) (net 23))
 (via (at 131.294 102.90188) (size 0.35) (drill 0.15) (layers F.Cu B.Cu) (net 23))
 (segment (start 131.294 97.096) (end 131.294 96.774) (width 0.2032) (layer B.Cu) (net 23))
 (via (at 131.294 97.096) (size 0.35) (drill 0.15) (layers F.Cu B.Cu) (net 23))
 (segment (start 131.694 102.19868) (end 131.694 96.774) (width 0.2032) (layer B.Cu) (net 24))
 (segment (start 131.694 102.90188) (end 131.694 102.576) (width 0.2032) (layer F.Cu) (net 24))
 (segment (start 131.694 102.576) (end 131.694 102.19868) (width 0.2032) (layer B.Cu) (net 24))
 (via (at 131.694 102.576) (size 0.35) (drill 0.15) (layers F.Cu B.Cu) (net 24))
 (segment (start 131.694 96.774) (end 131.694 96.774) (width 0.2032) (layer F.Cu) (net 24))
 (via (at 131.694 96.774) (size 0.35) (drill 0.15) (layers F.Cu B.Cu) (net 24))
 (segment (start 132.094 102.90188) (end 132.094 102.90188) (width 0.2032) (layer B.Cu) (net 25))
 (segment (start 132.094 102.90188) (end 132.094 97.106) (width 0.2032) (layer B.Cu) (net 25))
 (via (at 132.094 102.90188) (size 0.35) (drill 0.15) (layers F.Cu B.Cu) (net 25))
 (segment (start 132.094 97.106) (end 132.094 96.774) (width 0.2032) (layer B.Cu) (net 25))
 (via (at 132.094 97.106) (size 0.35) (drill 0.15) (layers F.Cu B.Cu) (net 25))
 (segment (start 132.494 102.90188) (end 132.494 102.576) (width 0.2032) (layer F.Cu) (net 26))
 (segment (start 132.494 102.576) (end 132.494 96.774) (width 0.2032) (layer B.Cu) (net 26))
 (via (at 132.494 102.576) (size 0.35) (drill 0.15) (layers F.Cu B.Cu) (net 26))
 (segment (start 132.494 96.774) (end 132.494 96.774) (width 0.2032) (layer F.Cu) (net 26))
 (via (at 132.494 96.774) (size 0.35) (drill 0.15) (layers F.Cu B.Cu) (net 26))
 (segment (start 132.894 102.19868) (end 132.894 97.096) (width 0.2032) (layer B.Cu) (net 27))
 (segment (start 132.894 102.90188) (end 132.894 102.90188) (width 0.2032) (layer B.Cu) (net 27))
 (segment (start 132.894 102.90188) (end 132.894 102.19868) (width 0.2032) (layer B.Cu) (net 27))
 (via (at 132.894 102.90188) (size 0.35) (drill 0.15) (layers F.Cu B.Cu) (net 27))
 (segment (start 132.894 97.096) (end 132.894 96.774) (width 0.2032) (layer B.Cu) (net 27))
 (via (at 132.894 97.096) (size 0.35) (drill 0.15) (layers F.Cu B.Cu) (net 27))
 (segment (start 133.294 102.19868) (end 133.294 96.774) (width 0.2032) (layer B.Cu) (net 28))
 (segment (start 133.294 102.90188) (end 133.294 102.576) (width 0.2032) (layer F.Cu) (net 28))
 (segment (start 133.294 102.576) (end 133.294 102.19868) (width 0.2032) (layer B.Cu) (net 28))
 (via (at 133.294 102.576) (size 0.35) (drill 0.15) (layers F.Cu B.Cu) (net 28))
 (segment (start 133.294 96.774) (end 133.294 96.774) (width 0.2032) (layer F.Cu) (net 28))
 (via (at 133.294 96.774) (size 0.35) (drill 0.15) (layers F.Cu B.Cu) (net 28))
 (segment (start 133.694 102.90188) (end 133.694 102.90188) (width 0.2032) (layer B.Cu) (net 29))
 (segment (start 133.694 102.90188) (end 133.694 97.096) (width 0.2032) (layer B.Cu) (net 29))
 (via (at 133.694 102.90188) (size 0.35) (drill 0.15) (layers F.Cu B.Cu) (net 29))
 (segment (start 133.694 97.096) (end 133.694 96.774) (width 0.2032) (layer B.Cu) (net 29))
 (via (at 133.694 97.096) (size 0.35) (drill 0.15) (layers F.Cu B.Cu) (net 29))
 (segment (start 134.094 102.19868) (end 134.094 96.774) (width 0.2032) (layer B.Cu) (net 30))
 (segment (start 134.094 102.90188) (end 134.094 102.576) (width 0.2032) (layer F.Cu) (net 30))
 (segment (start 134.094 102.576) (end 134.094 102.19868) (width 0.2032) (layer B.Cu) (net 30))
 (via (at 134.094 102.576) (size 0.35) (drill 0.15) (layers F.Cu B.Cu) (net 30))
 (segment (start 134.094 96.774) (end 134.094 96.774) (width 0.2032) (layer F.Cu) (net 30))
 (via (at 134.094 96.774) (size 0.35) (drill 0.15) (layers F.Cu B.Cu) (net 30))
 (segment (start 134.494 102.90188) (end 134.494 102.90188) (width 0.2032) (layer B.Cu) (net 31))
 (segment (start 134.494 102.90188) (end 134.494 97.096) (width 0.2032) (layer B.Cu) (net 31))
 (via (at 134.494 102.90188) (size 0.35) (drill 0.15) (layers F.Cu B.Cu) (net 31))
 (segment (start 134.494 97.096) (end 134.494 96.774) (width 0.2032) (layer B.Cu) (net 31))
 (via (at 134.494 97.096) (size 0.35) (drill 0.15) (layers F.Cu B.Cu) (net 31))
 (segment (start 134.894 102.90188) (end 134.894 102.576) (width 0.2032) (layer F.Cu) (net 32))
 (segment (start 134.894 102.576) (end 134.894 96.774) (width 0.2032) (layer B.Cu) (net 32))
 (via (at 134.894 102.576) (size 0.35) (drill 0.15) (layers F.Cu B.Cu) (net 32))
 (segment (start 134.894 96.774) (end 134.894 96.774) (width 0.2032) (layer F.Cu) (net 32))
 (via (at 134.894 96.774) (size 0.35) (drill 0.15) (layers F.Cu B.Cu) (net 32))
 (segment (start 135.294 102.19868) (end 135.294 97.096) (width 0.2032) (layer B.Cu) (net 33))
 (segment (start 135.294 102.90188) (end 135.294 102.90188) (width 0.2032) (layer B.Cu) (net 33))
 (segment (start 135.294 102.90188) (end 135.294 102.19868) (width 0.2032) (layer B.Cu) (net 33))
 (via (at 135.294 102.90188) (size 0.35) (drill 0.15) (layers F.Cu B.Cu) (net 33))
 (segment (start 135.294 97.096) (end 135.294 96.774) (width 0.2032) (layer B.Cu) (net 33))
 (via (at 135.294 97.096) (size 0.35) (drill 0.15) (layers F.Cu B.Cu) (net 33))
 (segment (start 142.76208 96.77686) (end 142.7634 96.77554) (width 0.2032) (layer F.Cu) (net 1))
 (segment (start 142.76208 103.5167) (end 142.76208 97.09808) (width 0.2032) (layer B.Cu) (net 1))
 (via (at 142.76208 103.5167) (size 0.35) (drill 0.15) (layers F.Cu B.Cu) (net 1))
 (segment (start 142.76208 97.09808) (end 142.76208 96.77686) (width 0.2032) (layer F.Cu) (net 1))
 (via (at 142.76208 97.09808) (size 0.35) (drill 0.15) (layers F.Cu B.Cu) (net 1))
 (segment (start 143.16208 96.77686) (end 143.1634 96.77554) (width 0.2032) (layer B.Cu) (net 2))
 (segment (start 143.16208 103.5167) (end 143.16208 103.18808) (width 0.2032) (layer B.Cu) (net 2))
 (via (at 143.1634 96.77554) (size 0.35) (drill 0.15) (layers F.Cu B.Cu) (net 2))
 (segment (start 143.16208 103.18808) (end 143.16208 96.77686) (width 0.2032) (layer B.Cu) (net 2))
 (via (at 143.16208 103.196) (size 0.35) (drill 0.15) (layers F.Cu B.Cu) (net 2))
 (segment (start 143.56208 96.77686) (end 143.5634 96.77554) (width 0.2032) (layer F.Cu) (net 3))
 (segment (start 143.56208 103.5167) (end 143.56208 97.09808) (width 0.2032) (layer B.Cu) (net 3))
 (via (at 143.56208 103.5167) (size 0.35) (drill 0.15) (layers F.Cu B.Cu) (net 3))
 (segment (start 143.56208 97.09808) (end 143.56208 96.77686) (width 0.2032) (layer F.Cu) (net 3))
 (via (at 143.56208 97.09808) (size 0.35) (drill 0.15) (layers F.Cu B.Cu) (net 3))
 (segment (start 143.96208 96.77686) (end 143.9634 96.77554) (width 0.2032) (layer B.Cu) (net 4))
 (segment (start 143.96208 103.5167) (end 143.96208 103.18808) (width 0.2032) (layer B.Cu) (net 4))
 (via (at 143.9634 96.77554) (size 0.35) (drill 0.15) (layers F.Cu B.Cu) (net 4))
 (segment (start 143.96208 103.18808) (end 143.96208 96.77686) (width 0.2032) (layer B.Cu) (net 4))
 (via (at 143.96208 103.196) (size 0.35) (drill 0.15) (layers F.Cu B.Cu) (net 4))
 (segment (start 144.36208 96.77686) (end 144.3634 96.77554) (width 0.2032) (layer F.Cu) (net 5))
 (segment (start 144.36208 103.5167) (end 144.36208 97.09808) (width 0.2032) (layer B.Cu) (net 5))
 (via (at 144.36208 103.5167) (size 0.35) (drill 0.15) (layers F.Cu B.Cu) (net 5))
 (segment (start 144.36208 97.09808) (end 144.36208 96.77686) (width 0.2032) (layer F.Cu) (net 5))
 (via (at 144.36208 97.09808) (size 0.35) (drill 0.15) (layers F.Cu B.Cu) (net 5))
 (segment (start 144.76208 96.77686) (end 144.7634 96.77554) (width 0.2032) (layer B.Cu) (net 6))
 (segment (start 144.76208 103.5167) (end 144.76208 103.19808) (width 0.2032) (layer B.Cu) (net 6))
 (via (at 144.7634 96.77554) (size 0.35) (drill 0.15) (layers F.Cu B.Cu) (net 6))
 (segment (start 144.76208 103.19808) (end 144.76208 96.77686) (width 0.2032) (layer B.Cu) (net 6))
 (via (at 144.76208 103.19808) (size 0.35) (drill 0.15) (layers F.Cu B.Cu) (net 6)))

